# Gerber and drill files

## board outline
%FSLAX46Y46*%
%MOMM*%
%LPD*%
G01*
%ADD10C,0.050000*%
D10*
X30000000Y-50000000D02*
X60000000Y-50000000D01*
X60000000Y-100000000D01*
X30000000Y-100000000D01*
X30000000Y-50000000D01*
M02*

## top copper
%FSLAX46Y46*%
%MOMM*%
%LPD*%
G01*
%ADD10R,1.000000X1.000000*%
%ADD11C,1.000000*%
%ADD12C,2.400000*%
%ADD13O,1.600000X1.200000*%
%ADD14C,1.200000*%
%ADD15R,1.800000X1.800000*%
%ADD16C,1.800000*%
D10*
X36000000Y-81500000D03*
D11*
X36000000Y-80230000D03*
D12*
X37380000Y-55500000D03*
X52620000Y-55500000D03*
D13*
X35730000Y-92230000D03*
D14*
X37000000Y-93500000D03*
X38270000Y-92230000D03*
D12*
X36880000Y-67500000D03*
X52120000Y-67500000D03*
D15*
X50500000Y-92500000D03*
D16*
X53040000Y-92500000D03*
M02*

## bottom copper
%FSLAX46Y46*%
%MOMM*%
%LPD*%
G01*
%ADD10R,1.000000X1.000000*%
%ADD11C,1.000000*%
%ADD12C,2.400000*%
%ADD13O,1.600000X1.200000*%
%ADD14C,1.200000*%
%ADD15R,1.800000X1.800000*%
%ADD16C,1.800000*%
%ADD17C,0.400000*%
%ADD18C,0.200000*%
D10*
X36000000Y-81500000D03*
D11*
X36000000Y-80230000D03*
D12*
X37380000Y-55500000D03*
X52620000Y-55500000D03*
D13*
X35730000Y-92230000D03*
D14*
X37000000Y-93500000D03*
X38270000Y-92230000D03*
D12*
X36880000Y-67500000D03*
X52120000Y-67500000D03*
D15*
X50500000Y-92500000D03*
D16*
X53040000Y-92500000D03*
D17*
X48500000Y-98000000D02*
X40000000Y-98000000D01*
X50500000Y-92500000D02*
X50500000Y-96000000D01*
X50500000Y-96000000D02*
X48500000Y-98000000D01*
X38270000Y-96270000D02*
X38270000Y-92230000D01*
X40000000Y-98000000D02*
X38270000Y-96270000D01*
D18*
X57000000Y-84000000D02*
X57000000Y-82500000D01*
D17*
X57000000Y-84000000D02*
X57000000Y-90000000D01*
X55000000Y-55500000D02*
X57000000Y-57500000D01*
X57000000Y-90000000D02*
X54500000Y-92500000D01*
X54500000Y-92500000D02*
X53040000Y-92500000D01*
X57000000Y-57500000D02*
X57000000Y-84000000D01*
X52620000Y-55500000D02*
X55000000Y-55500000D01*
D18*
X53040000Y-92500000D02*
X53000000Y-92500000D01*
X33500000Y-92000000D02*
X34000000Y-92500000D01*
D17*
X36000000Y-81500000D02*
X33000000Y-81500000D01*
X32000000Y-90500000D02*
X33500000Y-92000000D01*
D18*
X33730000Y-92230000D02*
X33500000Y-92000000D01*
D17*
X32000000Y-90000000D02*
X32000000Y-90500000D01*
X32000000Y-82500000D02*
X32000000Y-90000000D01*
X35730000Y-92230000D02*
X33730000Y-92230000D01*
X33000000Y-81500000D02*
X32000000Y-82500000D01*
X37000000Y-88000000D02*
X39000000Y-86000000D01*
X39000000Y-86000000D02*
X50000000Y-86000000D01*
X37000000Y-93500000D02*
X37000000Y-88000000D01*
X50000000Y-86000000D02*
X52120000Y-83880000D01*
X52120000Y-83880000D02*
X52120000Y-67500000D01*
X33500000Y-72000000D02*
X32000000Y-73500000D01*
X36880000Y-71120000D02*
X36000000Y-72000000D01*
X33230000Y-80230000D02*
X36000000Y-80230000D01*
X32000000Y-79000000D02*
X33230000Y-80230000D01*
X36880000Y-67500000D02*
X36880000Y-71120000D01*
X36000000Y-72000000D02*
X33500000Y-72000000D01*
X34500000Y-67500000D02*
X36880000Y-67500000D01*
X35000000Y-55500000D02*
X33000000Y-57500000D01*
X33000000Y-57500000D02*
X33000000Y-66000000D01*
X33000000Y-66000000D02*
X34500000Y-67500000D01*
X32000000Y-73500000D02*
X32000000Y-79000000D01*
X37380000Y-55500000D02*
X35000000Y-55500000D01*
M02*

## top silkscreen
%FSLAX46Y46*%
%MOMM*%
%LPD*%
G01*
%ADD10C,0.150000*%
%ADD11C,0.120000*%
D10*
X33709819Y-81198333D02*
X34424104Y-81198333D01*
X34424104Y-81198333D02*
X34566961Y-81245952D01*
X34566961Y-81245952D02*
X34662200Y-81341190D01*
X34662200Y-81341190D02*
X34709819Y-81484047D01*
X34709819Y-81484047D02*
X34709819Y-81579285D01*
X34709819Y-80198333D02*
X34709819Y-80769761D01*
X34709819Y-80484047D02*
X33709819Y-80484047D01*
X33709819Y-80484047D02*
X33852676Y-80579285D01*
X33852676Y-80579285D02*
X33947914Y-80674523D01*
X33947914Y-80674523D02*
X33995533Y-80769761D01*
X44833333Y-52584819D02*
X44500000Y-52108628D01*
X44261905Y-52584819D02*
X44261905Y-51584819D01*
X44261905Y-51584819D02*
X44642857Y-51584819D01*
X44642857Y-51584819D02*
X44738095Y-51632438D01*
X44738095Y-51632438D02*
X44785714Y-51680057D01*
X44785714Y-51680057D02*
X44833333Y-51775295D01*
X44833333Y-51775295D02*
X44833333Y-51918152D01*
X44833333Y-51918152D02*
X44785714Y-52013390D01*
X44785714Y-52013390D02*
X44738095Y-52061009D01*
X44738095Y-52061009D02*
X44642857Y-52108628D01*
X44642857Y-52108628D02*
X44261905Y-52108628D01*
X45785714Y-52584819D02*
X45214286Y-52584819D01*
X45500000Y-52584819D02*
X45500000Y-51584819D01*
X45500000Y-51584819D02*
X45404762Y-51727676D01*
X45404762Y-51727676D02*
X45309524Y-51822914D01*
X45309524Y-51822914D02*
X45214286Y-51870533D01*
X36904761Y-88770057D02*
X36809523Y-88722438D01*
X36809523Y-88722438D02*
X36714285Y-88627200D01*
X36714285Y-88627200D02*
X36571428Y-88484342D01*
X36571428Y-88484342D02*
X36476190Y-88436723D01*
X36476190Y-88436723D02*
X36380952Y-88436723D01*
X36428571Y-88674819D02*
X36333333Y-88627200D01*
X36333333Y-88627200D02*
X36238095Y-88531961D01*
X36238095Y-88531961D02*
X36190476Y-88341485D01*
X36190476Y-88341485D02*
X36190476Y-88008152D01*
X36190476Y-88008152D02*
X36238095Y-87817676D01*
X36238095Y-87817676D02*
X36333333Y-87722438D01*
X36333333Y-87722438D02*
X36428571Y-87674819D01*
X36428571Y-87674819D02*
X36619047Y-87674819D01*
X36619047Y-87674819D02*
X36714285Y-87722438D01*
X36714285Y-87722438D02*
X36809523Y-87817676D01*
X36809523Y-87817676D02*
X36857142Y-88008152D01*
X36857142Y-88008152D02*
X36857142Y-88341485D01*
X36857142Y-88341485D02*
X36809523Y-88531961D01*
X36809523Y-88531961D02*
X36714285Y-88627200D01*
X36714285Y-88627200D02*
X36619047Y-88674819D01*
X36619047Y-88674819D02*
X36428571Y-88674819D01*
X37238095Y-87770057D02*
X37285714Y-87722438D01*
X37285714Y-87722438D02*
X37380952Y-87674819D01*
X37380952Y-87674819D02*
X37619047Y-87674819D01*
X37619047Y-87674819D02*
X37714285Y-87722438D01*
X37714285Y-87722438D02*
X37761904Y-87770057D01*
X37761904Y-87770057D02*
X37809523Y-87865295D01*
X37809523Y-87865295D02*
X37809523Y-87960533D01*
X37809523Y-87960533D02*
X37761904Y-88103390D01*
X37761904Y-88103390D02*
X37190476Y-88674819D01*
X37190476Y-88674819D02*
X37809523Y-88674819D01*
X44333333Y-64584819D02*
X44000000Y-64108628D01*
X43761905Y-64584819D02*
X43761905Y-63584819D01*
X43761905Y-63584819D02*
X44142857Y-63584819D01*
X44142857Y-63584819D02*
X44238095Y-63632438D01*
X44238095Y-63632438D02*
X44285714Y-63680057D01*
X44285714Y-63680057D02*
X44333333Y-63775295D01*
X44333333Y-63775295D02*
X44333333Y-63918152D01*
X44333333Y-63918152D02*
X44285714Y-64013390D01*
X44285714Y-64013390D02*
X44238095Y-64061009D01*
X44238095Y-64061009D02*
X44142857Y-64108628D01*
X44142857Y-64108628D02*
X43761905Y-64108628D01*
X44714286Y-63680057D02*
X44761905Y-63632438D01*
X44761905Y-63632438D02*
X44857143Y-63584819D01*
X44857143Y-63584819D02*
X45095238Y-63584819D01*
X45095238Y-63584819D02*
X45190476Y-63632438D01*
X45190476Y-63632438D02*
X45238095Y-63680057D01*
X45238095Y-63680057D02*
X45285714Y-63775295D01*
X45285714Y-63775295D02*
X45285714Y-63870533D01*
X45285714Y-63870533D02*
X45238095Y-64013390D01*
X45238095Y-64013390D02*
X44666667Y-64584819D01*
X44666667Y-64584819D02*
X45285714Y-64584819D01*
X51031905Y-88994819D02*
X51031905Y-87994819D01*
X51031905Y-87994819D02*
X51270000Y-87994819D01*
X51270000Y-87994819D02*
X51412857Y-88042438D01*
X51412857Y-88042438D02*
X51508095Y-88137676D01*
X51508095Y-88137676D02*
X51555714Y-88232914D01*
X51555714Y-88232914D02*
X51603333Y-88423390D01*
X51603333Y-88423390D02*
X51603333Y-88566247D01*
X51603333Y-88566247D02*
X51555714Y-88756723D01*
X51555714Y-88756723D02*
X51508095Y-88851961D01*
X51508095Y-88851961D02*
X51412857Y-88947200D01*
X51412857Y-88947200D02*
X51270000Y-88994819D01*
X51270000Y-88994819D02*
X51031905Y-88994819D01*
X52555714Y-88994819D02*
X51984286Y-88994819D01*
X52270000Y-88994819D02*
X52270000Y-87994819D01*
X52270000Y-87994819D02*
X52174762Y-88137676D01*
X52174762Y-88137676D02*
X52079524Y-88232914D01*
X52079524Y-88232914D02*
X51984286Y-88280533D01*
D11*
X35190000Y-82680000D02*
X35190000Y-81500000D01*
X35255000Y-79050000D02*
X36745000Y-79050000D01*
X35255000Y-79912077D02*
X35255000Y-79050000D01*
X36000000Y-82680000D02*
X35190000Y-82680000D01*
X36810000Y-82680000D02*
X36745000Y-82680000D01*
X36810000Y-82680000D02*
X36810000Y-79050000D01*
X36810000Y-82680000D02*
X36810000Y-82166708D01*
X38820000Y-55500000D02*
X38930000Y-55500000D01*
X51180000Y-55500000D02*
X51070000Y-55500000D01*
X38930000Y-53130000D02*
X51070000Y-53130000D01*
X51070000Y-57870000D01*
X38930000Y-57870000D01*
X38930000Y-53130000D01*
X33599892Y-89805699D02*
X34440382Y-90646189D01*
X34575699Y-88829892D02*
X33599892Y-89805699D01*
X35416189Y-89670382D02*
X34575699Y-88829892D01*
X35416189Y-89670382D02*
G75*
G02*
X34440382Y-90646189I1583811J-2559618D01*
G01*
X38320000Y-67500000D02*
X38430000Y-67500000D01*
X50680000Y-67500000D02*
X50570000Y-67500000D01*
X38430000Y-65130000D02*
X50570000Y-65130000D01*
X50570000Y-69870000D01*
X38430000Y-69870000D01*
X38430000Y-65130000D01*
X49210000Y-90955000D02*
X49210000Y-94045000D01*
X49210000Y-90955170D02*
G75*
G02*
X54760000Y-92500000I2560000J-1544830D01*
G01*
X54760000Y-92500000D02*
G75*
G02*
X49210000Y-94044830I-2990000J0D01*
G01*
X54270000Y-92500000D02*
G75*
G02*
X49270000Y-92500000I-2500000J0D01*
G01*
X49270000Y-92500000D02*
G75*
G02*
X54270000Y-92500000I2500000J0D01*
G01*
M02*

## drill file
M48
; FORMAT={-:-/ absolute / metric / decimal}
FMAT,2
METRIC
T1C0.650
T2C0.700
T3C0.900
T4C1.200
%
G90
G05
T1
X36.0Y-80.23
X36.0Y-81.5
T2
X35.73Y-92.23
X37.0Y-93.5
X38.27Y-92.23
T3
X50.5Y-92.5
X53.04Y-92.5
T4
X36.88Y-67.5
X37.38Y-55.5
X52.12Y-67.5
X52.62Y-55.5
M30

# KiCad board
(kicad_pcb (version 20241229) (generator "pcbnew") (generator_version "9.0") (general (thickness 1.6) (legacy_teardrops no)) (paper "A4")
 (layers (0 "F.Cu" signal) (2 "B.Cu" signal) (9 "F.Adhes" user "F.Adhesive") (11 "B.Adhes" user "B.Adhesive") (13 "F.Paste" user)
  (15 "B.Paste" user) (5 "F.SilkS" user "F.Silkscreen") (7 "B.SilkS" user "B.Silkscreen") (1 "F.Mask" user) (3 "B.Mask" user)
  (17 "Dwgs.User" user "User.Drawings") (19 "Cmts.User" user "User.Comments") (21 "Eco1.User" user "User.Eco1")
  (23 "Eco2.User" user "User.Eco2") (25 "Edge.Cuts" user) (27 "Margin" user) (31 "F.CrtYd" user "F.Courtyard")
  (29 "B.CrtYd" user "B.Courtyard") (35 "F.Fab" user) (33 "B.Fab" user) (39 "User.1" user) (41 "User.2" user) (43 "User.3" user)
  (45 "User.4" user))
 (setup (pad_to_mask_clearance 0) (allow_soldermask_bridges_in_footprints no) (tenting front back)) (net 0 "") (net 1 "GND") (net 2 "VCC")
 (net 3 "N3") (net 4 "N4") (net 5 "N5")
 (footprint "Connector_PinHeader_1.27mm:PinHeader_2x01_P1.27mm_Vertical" (layer "F.Cu") (at 36 81.5 90)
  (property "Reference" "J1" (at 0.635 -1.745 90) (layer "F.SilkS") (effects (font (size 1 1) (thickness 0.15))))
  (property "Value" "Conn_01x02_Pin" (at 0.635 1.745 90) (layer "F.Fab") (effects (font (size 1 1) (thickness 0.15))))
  (fp_line (start -1.18 -0.81) (end 0 -0.81) (stroke (width 0.12) (type solid)) (layer "F.SilkS"))
  (fp_line (start 2.45 -0.745) (end 2.45 0.745) (stroke (width 0.12) (type solid)) (layer "F.SilkS"))
  (fp_line (start 1.587923 -0.745) (end 2.45 -0.745) (stroke (width 0.12) (type solid)) (layer "F.SilkS"))
  (fp_line (start -1.18 0) (end -1.18 -0.81) (stroke (width 0.12) (type solid)) (layer "F.SilkS"))
  (fp_line (start -1.18 0.81) (end -1.18 0.745) (stroke (width 0.12) (type solid)) (layer "F.SilkS"))
  (fp_line (start -1.18 0.81) (end 2.45 0.81) (stroke (width 0.12) (type solid)) (layer "F.SilkS"))
  (fp_line (start -1.18 0.81) (end -0.666708 0.81) (stroke (width 0.12) (type solid)) (layer "F.SilkS"))
  (pad "1" thru_hole rect (at 0 0 90) (size 1 1) (drill 0.65) (layers "*.Cu" "*.Mask") (remove_unused_layers no) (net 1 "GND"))
  (pad "2" thru_hole circle (at 1.27 0 90) (size 1 1) (drill 0.65) (layers "*.Cu" "*.Mask") (remove_unused_layers no) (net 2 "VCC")))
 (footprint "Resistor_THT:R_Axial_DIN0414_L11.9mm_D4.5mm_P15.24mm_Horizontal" (layer "F.Cu") (at 37.38 55.5)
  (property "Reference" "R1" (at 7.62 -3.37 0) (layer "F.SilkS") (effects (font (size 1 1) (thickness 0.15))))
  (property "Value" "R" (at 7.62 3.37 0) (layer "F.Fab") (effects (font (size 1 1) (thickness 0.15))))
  (fp_line (start 1.44 0) (end 1.55 0) (stroke (width 0.12) (type solid)) (layer "F.SilkS"))
  (fp_line (start 13.8 0) (end 13.69 0) (stroke (width 0.12) (type solid)) (layer "F.SilkS"))
  (fp_rect (start 1.55 -2.37) (end 13.69 2.37) (stroke (width 0.12) (type solid)) (fill no) (layer "F.SilkS"))
  (pad "1" thru_hole circle (at 0 0) (size 2.4 2.4) (drill 1.2) (layers "*.Cu" "*.Mask") (remove_unused_layers no) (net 2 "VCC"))
  (pad "2" thru_hole circle (at 15.24 0) (size 2.4 2.4) (drill 1.2) (layers "*.Cu" "*.Mask") (remove_unused_layers no) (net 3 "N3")))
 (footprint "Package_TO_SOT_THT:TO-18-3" (layer "F.Cu") (at 35.73 92.23)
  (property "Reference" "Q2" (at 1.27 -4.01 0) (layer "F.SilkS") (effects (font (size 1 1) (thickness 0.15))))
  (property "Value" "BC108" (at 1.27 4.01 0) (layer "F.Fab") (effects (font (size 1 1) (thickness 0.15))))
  (fp_line (start -2.130108 -2.424301) (end -1.289618 -1.583811) (stroke (width 0.12) (type solid)) (layer "F.SilkS"))
  (fp_line (start -1.154301 -3.400108) (end -2.130108 -2.424301) (stroke (width 0.12) (type solid)) (layer "F.SilkS"))
  (fp_line (start -0.313811 -2.559618) (end -1.154301 -3.400108) (stroke (width 0.12) (type solid)) (layer "F.SilkS"))
  (fp_arc (start -0.313811 -2.559618) (mid 3.398391 2.128391) (end -1.289618 -1.583811) (stroke (width 0.12) (type solid)) (layer "F.SilkS"))
  (pad "1" thru_hole oval (at 0 0) (size 1.6 1.2) (drill 0.7) (layers "*.Cu" "*.Mask") (remove_unused_layers no) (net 1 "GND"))
  (pad "2" thru_hole circle (at 1.27 1.27) (size 1.2 1.2) (drill 0.7) (layers "*.Cu" "*.Mask") (remove_unused_layers no) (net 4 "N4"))
  (pad "3" thru_hole circle (at 2.54 0) (size 1.2 1.2) (drill 0.7) (layers "*.Cu" "*.Mask") (remove_unused_layers no) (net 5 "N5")))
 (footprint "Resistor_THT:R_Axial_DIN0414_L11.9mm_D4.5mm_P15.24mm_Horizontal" (layer "F.Cu") (at 36.88 67.5)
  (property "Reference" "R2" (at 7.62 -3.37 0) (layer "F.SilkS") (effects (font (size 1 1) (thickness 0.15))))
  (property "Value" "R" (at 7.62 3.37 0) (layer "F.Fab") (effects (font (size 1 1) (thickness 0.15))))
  (fp_line (start 1.44 0) (end 1.55 0) (stroke (width 0.12) (type solid)) (layer "F.SilkS"))
  (fp_line (start 13.8 0) (end 13.69 0) (stroke (width 0.12) (type solid)) (layer "F.SilkS"))
  (fp_rect (start 1.55 -2.37) (end 13.69 2.37) (stroke (width 0.12) (type solid)) (fill no) (layer "F.SilkS"))
  (pad "1" thru_hole circle (at 0 0) (size 2.4 2.4) (drill 1.2) (layers "*.Cu" "*.Mask") (remove_unused_layers no) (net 2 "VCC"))
  (pad "2" thru_hole circle (at 15.24 0) (size 2.4 2.4) (drill 1.2) (layers "*.Cu" "*.Mask") (remove_unused_layers no) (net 4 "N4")))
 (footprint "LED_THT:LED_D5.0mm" (layer "F.Cu") (at 50.5 92.5)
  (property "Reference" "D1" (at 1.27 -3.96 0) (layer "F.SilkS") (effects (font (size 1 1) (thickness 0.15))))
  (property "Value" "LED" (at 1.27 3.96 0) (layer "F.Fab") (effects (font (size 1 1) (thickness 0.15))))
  (fp_line (start -1.29 -1.545) (end -1.29 1.545) (stroke (width 0.12) (type solid)) (layer "F.SilkS"))
  (fp_arc (start -1.29 -1.54483) (mid 2.071779 -2.880495) (end 4.26 0) (stroke (width 0.12) (type solid)) (layer "F.SilkS"))
  (fp_arc (start 4.26 0) (mid 2.071779 2.880495) (end -1.29 1.54483) (stroke (width 0.12) (type solid)) (layer "F.SilkS"))
  (fp_circle (center 1.27 0) (end 3.77 0) (stroke (width 0.12) (type solid)) (fill no) (layer "F.SilkS"))
  (pad "1" thru_hole rect (at 0 0) (size 1.8 1.8) (drill 0.9) (layers "*.Cu" "*.Mask") (remove_unused_layers no) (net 5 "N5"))
  (pad "2" thru_hole circle (at 2.54 0) (size 1.8 1.8) (drill 0.9) (layers "*.Cu" "*.Mask") (remove_unused_layers no) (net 3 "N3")))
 (gr_rect (start 30 50) (end 60 100) (stroke (width 0.05) (type solid)) (fill no) (layer "Edge.Cuts"))
 (segment (start 48.5 98) (end 40 98) (width 0.4) (layer "B.Cu") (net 5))
 (segment (start 50.5 92.5) (end 50.5 96) (width 0.4) (layer "B.Cu") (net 5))
 (segment (start 50.5 96) (end 48.5 98) (width 0.4) (layer "B.Cu") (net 5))
 (segment (start 38.27 96.27) (end 38.27 92.23) (width 0.4) (layer "B.Cu") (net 5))
 (segment (start 40 98) (end 38.27 96.27) (width 0.4) (layer "B.Cu") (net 5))
 (segment (start 57 84) (end 57 82.5) (width 0.2) (layer "B.Cu") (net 3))
 (segment (start 57 84) (end 57 90) (width 0.4) (layer "B.Cu") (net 3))
 (segment (start 55 55.5) (end 57 57.5) (width 0.4) (layer "B.Cu") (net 3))
 (segment (start 57 90) (end 54.5 92.5) (width 0.4) (layer "B.Cu") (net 3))
 (segment (start 54.5 92.5) (end 53.04 92.5) (width 0.4) (layer "B.Cu") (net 3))
 (segment (start 57 57.5) (end 57 84) (width 0.4) (layer "B.Cu") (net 3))
 (segment (start 52.62 55.5) (end 55 55.5) (width 0.4) (layer "B.Cu") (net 3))
 (segment (start 53.04 92.5) (end 53 92.5) (width 0.2) (layer "B.Cu") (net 3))
 (segment (start 33.5 92) (end 34 92.5) (width 0.2) (layer "B.Cu") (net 1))
 (segment (start 36 81.5) (end 33 81.5) (width 0.4) (layer "B.Cu") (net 1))
 (segment (start 32 90.5) (end 33.5 92) (width 0.4) (layer "B.Cu") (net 1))
 (segment (start 33.73 92.23) (end 33.5 92) (width 0.2) (layer "B.Cu") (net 1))
 (segment (start 32 90) (end 32 90.5) (width 0.4) (layer "B.Cu") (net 1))
 (segment (start 32 82.5) (end 32 90) (width 0.4) (layer "B.Cu") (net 1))
 (segment (start 35.73 92.23) (end 33.73 92.23) (width 0.4) (layer "B.Cu") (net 1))
 (segment (start 33 81.5) (end 32 82.5) (width 0.4) (layer "B.Cu") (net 1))
 (segment (start 37 88) (end 39 86) (width 0.4) (layer "B.Cu") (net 4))
 (segment (start 39 86) (end 50 86) (width 0.4) (layer "B.Cu") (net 4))
 (segment (start 37 93.5) (end 37 88) (width 0.4) (layer "B.Cu") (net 4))
 (segment (start 50 86) (end 52.12 83.88) (width 0.4) (layer "B.Cu") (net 4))
 (segment (start 52.12 83.88) (end 52.12 67.5) (width 0.4) (layer "B.Cu") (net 4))
 (segment (start 33.5 72) (end 32 73.5) (width 0.4) (layer "B.Cu") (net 2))
 (segment (start 36.88 71.12) (end 36 72) (width 0.4) (layer "B.Cu") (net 2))
 (segment (start 33.23 80.23) (end 36 80.23) (width 0.4) (layer "B.Cu") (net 2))
 (segment (start 32 79) (end 33.23 80.23) (width 0.4) (layer "B.Cu") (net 2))
 (segment (start 36.88 67.5) (end 36.88 71.12) (width 0.4) (layer "B.Cu") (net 2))
 (segment (start 36 72) (end 33.5 72) (width 0.4) (layer "B.Cu") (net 2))
 (segment (start 34.5 67.5) (end 36.88 67.5) (width 0.4) (layer "B.Cu") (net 2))
 (segment (start 35 55.5) (end 33 57.5) (width 0.4) (layer "B.Cu") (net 2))
 (segment (start 33 57.5) (end 33 66) (width 0.4) (layer "B.Cu") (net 2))
 (segment (start 33 66) (end 34.5 67.5) (width 0.4) (layer "B.Cu") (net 2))
 (segment (start 32 73.5) (end 32 79) (width 0.4) (layer "B.Cu") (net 2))
 (segment (start 37.38 55.5) (end 35 55.5) (width 0.4) (layer "B.Cu") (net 2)))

